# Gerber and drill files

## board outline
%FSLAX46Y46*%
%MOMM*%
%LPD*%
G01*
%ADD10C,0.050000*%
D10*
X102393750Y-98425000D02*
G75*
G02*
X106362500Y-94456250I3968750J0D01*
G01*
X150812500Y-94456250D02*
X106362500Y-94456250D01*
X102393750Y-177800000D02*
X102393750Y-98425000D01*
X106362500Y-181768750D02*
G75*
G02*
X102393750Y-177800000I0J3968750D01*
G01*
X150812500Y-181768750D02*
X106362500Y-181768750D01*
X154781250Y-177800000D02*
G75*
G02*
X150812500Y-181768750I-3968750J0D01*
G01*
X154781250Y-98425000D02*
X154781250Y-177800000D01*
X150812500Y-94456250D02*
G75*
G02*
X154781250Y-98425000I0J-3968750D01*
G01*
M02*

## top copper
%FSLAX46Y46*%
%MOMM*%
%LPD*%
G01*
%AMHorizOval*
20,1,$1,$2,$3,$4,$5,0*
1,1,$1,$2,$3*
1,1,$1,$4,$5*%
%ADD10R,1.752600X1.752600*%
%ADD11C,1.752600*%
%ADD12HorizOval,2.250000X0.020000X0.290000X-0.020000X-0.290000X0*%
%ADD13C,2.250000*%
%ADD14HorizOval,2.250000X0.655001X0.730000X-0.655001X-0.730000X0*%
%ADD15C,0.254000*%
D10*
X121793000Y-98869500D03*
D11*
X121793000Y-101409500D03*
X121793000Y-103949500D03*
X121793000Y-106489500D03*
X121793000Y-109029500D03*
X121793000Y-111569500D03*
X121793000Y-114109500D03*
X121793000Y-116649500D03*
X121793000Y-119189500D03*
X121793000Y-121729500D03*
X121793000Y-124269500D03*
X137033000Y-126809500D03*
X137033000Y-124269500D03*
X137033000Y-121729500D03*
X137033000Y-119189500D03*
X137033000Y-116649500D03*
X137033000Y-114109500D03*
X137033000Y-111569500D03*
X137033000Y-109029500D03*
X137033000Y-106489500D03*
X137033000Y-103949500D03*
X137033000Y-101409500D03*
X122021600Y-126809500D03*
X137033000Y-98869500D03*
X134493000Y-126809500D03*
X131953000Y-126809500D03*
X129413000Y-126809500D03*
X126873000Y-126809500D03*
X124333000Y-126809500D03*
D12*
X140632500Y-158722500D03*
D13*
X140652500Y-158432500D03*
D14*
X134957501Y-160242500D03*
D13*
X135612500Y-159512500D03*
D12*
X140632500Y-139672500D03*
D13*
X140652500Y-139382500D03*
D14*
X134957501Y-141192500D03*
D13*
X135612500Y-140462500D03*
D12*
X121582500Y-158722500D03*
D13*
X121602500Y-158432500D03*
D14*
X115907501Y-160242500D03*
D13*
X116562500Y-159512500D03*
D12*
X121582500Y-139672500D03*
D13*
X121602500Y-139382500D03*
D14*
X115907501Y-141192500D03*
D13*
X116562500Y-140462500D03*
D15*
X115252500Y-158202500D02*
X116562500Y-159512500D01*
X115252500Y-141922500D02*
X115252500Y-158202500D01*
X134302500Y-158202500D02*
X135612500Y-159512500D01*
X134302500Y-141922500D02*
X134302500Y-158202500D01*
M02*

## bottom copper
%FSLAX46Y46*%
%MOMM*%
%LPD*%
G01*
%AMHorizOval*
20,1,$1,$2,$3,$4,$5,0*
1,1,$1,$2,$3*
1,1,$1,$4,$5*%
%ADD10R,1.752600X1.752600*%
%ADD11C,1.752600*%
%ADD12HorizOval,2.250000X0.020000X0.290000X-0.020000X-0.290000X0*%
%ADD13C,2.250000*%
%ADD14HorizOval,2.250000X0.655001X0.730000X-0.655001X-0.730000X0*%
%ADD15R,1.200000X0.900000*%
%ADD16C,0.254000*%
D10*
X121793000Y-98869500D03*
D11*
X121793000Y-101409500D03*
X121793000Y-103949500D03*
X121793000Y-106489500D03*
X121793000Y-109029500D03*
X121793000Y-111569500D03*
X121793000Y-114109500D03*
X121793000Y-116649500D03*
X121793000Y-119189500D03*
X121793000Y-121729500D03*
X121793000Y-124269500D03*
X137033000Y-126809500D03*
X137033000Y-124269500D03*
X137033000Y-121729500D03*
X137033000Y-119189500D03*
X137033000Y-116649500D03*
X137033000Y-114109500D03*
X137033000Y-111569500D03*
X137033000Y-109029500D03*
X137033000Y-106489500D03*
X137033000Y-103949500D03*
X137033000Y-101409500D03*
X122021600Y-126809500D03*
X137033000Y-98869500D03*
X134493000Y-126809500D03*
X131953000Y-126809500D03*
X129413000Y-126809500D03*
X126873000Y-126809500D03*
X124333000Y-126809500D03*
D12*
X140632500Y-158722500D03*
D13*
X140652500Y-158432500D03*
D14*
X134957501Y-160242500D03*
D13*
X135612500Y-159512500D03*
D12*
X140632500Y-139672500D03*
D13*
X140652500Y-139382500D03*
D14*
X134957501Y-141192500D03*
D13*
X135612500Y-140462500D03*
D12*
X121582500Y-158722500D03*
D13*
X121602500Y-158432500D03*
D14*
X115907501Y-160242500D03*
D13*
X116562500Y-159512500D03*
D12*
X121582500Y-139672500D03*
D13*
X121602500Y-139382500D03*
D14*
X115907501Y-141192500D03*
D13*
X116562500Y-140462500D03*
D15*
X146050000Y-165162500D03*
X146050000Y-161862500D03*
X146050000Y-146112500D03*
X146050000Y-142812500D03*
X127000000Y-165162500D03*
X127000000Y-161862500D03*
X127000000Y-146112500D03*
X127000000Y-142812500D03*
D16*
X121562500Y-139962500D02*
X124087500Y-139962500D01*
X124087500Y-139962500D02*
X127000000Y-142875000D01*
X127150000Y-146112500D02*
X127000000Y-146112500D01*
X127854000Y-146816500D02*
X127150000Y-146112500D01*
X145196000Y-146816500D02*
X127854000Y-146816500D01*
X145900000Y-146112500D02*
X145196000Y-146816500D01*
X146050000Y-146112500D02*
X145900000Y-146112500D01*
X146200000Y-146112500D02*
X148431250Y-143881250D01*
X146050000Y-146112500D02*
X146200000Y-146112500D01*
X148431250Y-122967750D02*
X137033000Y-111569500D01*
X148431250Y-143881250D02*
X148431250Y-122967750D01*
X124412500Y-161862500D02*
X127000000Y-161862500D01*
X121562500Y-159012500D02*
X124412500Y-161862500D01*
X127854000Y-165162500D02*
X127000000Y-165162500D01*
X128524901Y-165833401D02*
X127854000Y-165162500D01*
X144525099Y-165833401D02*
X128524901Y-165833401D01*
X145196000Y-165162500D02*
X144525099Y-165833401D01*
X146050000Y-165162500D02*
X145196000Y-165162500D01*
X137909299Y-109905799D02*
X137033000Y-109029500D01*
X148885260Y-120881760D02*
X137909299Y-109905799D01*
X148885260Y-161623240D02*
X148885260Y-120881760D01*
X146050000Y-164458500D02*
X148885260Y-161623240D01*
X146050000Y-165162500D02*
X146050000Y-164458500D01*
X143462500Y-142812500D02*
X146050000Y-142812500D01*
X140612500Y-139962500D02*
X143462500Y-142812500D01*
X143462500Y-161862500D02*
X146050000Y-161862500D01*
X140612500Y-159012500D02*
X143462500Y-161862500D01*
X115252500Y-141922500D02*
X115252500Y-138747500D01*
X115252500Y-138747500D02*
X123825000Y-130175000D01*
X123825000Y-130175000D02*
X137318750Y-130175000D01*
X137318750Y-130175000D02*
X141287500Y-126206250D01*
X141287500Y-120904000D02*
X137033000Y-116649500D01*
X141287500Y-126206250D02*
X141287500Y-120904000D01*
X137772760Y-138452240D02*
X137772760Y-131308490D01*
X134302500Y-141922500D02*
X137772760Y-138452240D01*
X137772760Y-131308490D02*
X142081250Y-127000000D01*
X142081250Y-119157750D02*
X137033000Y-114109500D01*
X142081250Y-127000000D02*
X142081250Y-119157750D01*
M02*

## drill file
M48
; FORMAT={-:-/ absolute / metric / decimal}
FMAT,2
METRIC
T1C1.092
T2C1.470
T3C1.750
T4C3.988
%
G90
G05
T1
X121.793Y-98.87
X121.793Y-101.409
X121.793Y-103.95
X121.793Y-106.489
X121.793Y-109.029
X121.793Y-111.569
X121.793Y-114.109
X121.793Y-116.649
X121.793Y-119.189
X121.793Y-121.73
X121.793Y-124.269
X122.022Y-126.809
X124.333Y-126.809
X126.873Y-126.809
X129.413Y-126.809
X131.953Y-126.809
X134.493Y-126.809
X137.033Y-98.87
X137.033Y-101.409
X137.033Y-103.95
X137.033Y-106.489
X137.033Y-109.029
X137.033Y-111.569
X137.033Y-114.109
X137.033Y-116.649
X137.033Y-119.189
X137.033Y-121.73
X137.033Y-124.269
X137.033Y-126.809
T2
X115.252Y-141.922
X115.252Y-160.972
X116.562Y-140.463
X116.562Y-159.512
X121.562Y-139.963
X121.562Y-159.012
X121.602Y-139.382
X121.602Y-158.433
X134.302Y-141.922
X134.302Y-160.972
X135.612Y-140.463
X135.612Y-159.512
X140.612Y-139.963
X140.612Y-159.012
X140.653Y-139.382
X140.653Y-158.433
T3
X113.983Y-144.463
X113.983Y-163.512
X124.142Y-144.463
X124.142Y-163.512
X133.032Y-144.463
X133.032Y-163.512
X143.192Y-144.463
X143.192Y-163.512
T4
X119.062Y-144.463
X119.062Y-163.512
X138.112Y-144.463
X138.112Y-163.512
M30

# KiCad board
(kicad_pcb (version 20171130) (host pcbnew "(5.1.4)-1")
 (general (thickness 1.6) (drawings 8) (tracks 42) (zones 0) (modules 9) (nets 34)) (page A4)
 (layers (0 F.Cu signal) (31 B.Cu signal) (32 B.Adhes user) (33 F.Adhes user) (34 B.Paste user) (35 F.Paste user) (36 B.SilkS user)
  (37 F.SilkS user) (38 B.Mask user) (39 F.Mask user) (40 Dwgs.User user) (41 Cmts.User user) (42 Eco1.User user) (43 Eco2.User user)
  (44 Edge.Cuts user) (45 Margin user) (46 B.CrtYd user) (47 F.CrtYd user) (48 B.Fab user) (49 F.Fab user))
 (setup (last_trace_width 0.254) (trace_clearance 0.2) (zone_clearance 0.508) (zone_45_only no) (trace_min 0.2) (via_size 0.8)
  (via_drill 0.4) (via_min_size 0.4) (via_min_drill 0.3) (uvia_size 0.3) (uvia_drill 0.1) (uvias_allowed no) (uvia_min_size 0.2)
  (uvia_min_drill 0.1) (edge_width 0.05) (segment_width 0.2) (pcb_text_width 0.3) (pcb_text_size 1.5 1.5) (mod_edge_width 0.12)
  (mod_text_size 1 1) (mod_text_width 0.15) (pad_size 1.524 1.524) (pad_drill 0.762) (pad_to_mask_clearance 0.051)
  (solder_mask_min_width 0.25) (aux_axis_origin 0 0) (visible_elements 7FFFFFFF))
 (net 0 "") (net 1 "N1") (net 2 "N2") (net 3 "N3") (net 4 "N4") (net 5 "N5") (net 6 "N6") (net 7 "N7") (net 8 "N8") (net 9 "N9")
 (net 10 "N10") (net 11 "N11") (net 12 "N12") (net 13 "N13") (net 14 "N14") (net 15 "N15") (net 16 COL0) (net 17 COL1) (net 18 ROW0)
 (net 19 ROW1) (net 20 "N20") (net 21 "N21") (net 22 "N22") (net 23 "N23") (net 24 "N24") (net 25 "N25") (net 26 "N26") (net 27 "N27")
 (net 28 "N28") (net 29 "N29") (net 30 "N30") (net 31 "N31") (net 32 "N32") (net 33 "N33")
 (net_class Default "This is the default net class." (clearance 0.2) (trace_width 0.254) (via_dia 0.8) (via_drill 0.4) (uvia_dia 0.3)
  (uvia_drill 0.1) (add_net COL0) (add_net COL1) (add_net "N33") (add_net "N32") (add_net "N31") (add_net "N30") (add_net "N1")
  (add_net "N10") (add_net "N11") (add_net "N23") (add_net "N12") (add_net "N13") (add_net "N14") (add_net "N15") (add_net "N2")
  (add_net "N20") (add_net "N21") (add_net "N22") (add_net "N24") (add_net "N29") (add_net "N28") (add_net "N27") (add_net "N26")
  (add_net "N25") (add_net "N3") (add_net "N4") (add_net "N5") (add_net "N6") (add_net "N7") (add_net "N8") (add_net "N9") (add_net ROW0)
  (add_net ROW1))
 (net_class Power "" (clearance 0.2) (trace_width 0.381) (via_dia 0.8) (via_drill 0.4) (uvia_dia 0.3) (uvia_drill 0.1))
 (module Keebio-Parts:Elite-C (layer F.Cu) (at 129.413 112.8395 270)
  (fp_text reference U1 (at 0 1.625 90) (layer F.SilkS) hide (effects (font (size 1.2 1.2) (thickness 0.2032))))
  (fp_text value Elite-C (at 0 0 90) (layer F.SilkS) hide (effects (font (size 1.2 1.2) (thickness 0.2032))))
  (pad 1 thru_hole rect (at -13.97 7.62 270) (size 1.7526 1.7526) (drill 1.0922) (layers *.Cu *.SilkS *.Mask) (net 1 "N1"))
  (pad 2 thru_hole circle (at -11.43 7.62 270) (size 1.7526 1.7526) (drill 1.0922) (layers *.Cu *.SilkS *.Mask) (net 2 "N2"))
  (pad 3 thru_hole circle (at -8.89 7.62 270) (size 1.7526 1.7526) (drill 1.0922) (layers *.Cu *.SilkS *.Mask) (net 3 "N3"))
  (pad 4 thru_hole circle (at -6.35 7.62 270) (size 1.7526 1.7526) (drill 1.0922) (layers *.Cu *.SilkS *.Mask) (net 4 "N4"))
  (pad 5 thru_hole circle (at -3.81 7.62 270) (size 1.7526 1.7526) (drill 1.0922) (layers *.Cu *.SilkS *.Mask) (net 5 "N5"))
  (pad 6 thru_hole circle (at -1.27 7.62 270) (size 1.7526 1.7526) (drill 1.0922) (layers *.Cu *.SilkS *.Mask) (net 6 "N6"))
  (pad 7 thru_hole circle (at 1.27 7.62 270) (size 1.7526 1.7526) (drill 1.0922) (layers *.Cu *.SilkS *.Mask) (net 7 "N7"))
  (pad 8 thru_hole circle (at 3.81 7.62 270) (size 1.7526 1.7526) (drill 1.0922) (layers *.Cu *.SilkS *.Mask) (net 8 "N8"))
  (pad 9 thru_hole circle (at 6.35 7.62 270) (size 1.7526 1.7526) (drill 1.0922) (layers *.Cu *.SilkS *.Mask) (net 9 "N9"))
  (pad 10 thru_hole circle (at 8.89 7.62 270) (size 1.7526 1.7526) (drill 1.0922) (layers *.Cu *.SilkS *.Mask) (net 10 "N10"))
  (pad 11 thru_hole circle (at 11.43 7.62 270) (size 1.7526 1.7526) (drill 1.0922) (layers *.Cu *.SilkS *.Mask) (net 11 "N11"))
  (pad 13 thru_hole circle (at 13.97 -7.62 270) (size 1.7526 1.7526) (drill 1.0922) (layers *.Cu *.SilkS *.Mask) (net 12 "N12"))
  (pad 14 thru_hole circle (at 11.43 -7.62 270) (size 1.7526 1.7526) (drill 1.0922) (layers *.Cu *.SilkS *.Mask) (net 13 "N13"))
  (pad 15 thru_hole circle (at 8.89 -7.62 270) (size 1.7526 1.7526) (drill 1.0922) (layers *.Cu *.SilkS *.Mask) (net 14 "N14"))
  (pad 16 thru_hole circle (at 6.35 -7.62 270) (size 1.7526 1.7526) (drill 1.0922) (layers *.Cu *.SilkS *.Mask) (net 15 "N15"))
  (pad 17 thru_hole circle (at 3.81 -7.62 270) (size 1.7526 1.7526) (drill 1.0922) (layers *.Cu *.SilkS *.Mask) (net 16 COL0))
  (pad 18 thru_hole circle (at 1.27 -7.62 270) (size 1.7526 1.7526) (drill 1.0922) (layers *.Cu *.SilkS *.Mask) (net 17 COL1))
  (pad 19 thru_hole circle (at -1.27 -7.62 270) (size 1.7526 1.7526) (drill 1.0922) (layers *.Cu *.SilkS *.Mask) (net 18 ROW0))
  (pad 20 thru_hole circle (at -3.81 -7.62 270) (size 1.7526 1.7526) (drill 1.0922) (layers *.Cu *.SilkS *.Mask) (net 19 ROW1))
  (pad 21 thru_hole circle (at -6.35 -7.62 270) (size 1.7526 1.7526) (drill 1.0922) (layers *.Cu *.SilkS *.Mask) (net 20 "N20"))
  (pad 22 thru_hole circle (at -8.89 -7.62 270) (size 1.7526 1.7526) (drill 1.0922) (layers *.Cu *.SilkS *.Mask) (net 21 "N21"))
  (pad 23 thru_hole circle (at -11.43 -7.62 270) (size 1.7526 1.7526) (drill 1.0922) (layers *.Cu *.SilkS *.Mask) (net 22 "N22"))
  (pad 12 thru_hole circle (at 13.97 7.3914 270) (size 1.7526 1.7526) (drill 1.0922) (layers *.Cu *.SilkS *.Mask) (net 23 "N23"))
  (pad 24 thru_hole circle (at -13.97 -7.62 270) (size 1.7526 1.7526) (drill 1.0922) (layers *.Cu *.SilkS *.Mask) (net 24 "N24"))
  (pad 29 thru_hole circle (at 13.97 -5.08 270) (size 1.7526 1.7526) (drill 1.0922) (layers *.Cu *.SilkS *.Mask) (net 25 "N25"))
  (pad 28 thru_hole circle (at 13.97 -2.54 270) (size 1.7526 1.7526) (drill 1.0922) (layers *.Cu *.SilkS *.Mask) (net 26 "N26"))
  (pad 27 thru_hole circle (at 13.97 0 270) (size 1.7526 1.7526) (drill 1.0922) (layers *.Cu *.SilkS *.Mask) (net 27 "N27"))
  (pad 26 thru_hole circle (at 13.97 2.54 270) (size 1.7526 1.7526) (drill 1.0922) (layers *.Cu *.SilkS *.Mask) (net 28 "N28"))
  (pad 25 thru_hole circle (at 13.97 5.08 270) (size 1.7526 1.7526) (drill 1.0922) (layers *.Cu *.SilkS *.Mask) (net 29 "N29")))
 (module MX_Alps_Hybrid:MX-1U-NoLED (layer F.Cu) (at 138.1125 163.5125)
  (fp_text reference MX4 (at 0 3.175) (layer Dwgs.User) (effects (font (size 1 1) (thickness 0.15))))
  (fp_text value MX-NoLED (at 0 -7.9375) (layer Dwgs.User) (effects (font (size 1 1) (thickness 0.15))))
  (pad 2 thru_hole oval (at 2.5 -4.5 86.0548) (size 2.831378 2.25) (drill 1.47 (offset 0.290689 0)) (layers *.Cu B.Mask) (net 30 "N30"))
  (pad 2 thru_hole circle (at 2.54 -5.08) (size 2.25 2.25) (drill 1.47) (layers *.Cu B.Mask) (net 30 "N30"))
  (pad 1 thru_hole oval (at -3.81 -2.54 48.0996) (size 4.211556 2.25) (drill 1.47 (offset 0.980778 0)) (layers *.Cu B.Mask) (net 17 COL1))
  (pad "" np_thru_hole circle (at 0 0) (size 3.9878 3.9878) (drill 3.9878) (layers *.Cu *.Mask))
  (pad 1 thru_hole circle (at -2.5 -4) (size 2.25 2.25) (drill 1.47) (layers *.Cu B.Mask) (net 17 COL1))
  (pad "" np_thru_hole circle (at -5.08 0 48.0996) (size 1.75 1.75) (drill 1.75) (layers *.Cu *.Mask))
  (pad "" np_thru_hole circle (at 5.08 0 48.0996) (size 1.75 1.75) (drill 1.75) (layers *.Cu *.Mask)))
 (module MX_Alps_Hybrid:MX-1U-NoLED (layer F.Cu) (at 138.1125 144.4625)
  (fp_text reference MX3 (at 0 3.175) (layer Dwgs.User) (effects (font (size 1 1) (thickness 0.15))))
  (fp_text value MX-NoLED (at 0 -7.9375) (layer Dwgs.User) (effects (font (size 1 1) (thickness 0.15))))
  (pad 2 thru_hole oval (at 2.5 -4.5 86.0548) (size 2.831378 2.25) (drill 1.47 (offset 0.290689 0)) (layers *.Cu B.Mask) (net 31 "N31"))
  (pad 2 thru_hole circle (at 2.54 -5.08) (size 2.25 2.25) (drill 1.47) (layers *.Cu B.Mask) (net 31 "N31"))
  (pad 1 thru_hole oval (at -3.81 -2.54 48.0996) (size 4.211556 2.25) (drill 1.47 (offset 0.980778 0)) (layers *.Cu B.Mask) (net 17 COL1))
  (pad "" np_thru_hole circle (at 0 0) (size 3.9878 3.9878) (drill 3.9878) (layers *.Cu *.Mask))
  (pad 1 thru_hole circle (at -2.5 -4) (size 2.25 2.25) (drill 1.47) (layers *.Cu B.Mask) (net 17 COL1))
  (pad "" np_thru_hole circle (at -5.08 0 48.0996) (size 1.75 1.75) (drill 1.75) (layers *.Cu *.Mask))
  (pad "" np_thru_hole circle (at 5.08 0 48.0996) (size 1.75 1.75) (drill 1.75) (layers *.Cu *.Mask)))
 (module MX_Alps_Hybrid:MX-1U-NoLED (layer F.Cu) (at 119.0625 163.5125)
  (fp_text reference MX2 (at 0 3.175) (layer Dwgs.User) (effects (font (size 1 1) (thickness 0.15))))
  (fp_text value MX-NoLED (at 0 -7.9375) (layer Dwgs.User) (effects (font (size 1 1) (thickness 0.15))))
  (pad 2 thru_hole oval (at 2.5 -4.5 86.0548) (size 2.831378 2.25) (drill 1.47 (offset 0.290689 0)) (layers *.Cu B.Mask) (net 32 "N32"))
  (pad 2 thru_hole circle (at 2.54 -5.08) (size 2.25 2.25) (drill 1.47) (layers *.Cu B.Mask) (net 32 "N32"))
  (pad 1 thru_hole oval (at -3.81 -2.54 48.0996) (size 4.211556 2.25) (drill 1.47 (offset 0.980778 0)) (layers *.Cu B.Mask) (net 16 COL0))
  (pad "" np_thru_hole circle (at 0 0) (size 3.9878 3.9878) (drill 3.9878) (layers *.Cu *.Mask))
  (pad 1 thru_hole circle (at -2.5 -4) (size 2.25 2.25) (drill 1.47) (layers *.Cu B.Mask) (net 16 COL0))
  (pad "" np_thru_hole circle (at -5.08 0 48.0996) (size 1.75 1.75) (drill 1.75) (layers *.Cu *.Mask))
  (pad "" np_thru_hole circle (at 5.08 0 48.0996) (size 1.75 1.75) (drill 1.75) (layers *.Cu *.Mask)))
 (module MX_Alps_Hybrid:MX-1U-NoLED (layer F.Cu) (at 119.0625 144.4625)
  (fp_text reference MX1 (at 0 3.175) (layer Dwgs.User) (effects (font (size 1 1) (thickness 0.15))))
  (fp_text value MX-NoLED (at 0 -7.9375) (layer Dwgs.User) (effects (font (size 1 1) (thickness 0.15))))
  (pad 2 thru_hole oval (at 2.5 -4.5 86.0548) (size 2.831378 2.25) (drill 1.47 (offset 0.290689 0)) (layers *.Cu B.Mask) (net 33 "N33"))
  (pad 2 thru_hole circle (at 2.54 -5.08) (size 2.25 2.25) (drill 1.47) (layers *.Cu B.Mask) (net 33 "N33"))
  (pad 1 thru_hole oval (at -3.81 -2.54 48.0996) (size 4.211556 2.25) (drill 1.47 (offset 0.980778 0)) (layers *.Cu B.Mask) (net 16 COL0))
  (pad "" np_thru_hole circle (at 0 0) (size 3.9878 3.9878) (drill 3.9878) (layers *.Cu *.Mask))
  (pad 1 thru_hole circle (at -2.5 -4) (size 2.25 2.25) (drill 1.47) (layers *.Cu B.Mask) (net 16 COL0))
  (pad "" np_thru_hole circle (at -5.08 0 48.0996) (size 1.75 1.75) (drill 1.75) (layers *.Cu *.Mask))
  (pad "" np_thru_hole circle (at 5.08 0 48.0996) (size 1.75 1.75) (drill 1.75) (layers *.Cu *.Mask)))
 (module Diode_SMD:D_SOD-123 (layer B.Cu) (at 146.05 163.5125 90)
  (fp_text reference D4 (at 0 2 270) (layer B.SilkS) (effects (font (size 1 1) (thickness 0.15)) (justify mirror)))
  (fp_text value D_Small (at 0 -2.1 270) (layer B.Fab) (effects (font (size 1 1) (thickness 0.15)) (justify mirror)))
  (pad 1 smd rect (at -1.65 0 90) (size 0.9 1.2) (layers B.Cu B.Paste B.Mask) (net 19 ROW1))
  (pad 2 smd rect (at 1.65 0 90) (size 0.9 1.2) (layers B.Cu B.Paste B.Mask) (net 30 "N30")))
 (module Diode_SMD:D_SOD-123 (layer B.Cu) (at 146.05 144.4625 90)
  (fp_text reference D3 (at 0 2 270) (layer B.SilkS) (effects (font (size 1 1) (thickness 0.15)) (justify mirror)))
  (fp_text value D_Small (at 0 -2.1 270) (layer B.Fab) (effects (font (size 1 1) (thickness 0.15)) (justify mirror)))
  (pad 1 smd rect (at -1.65 0 90) (size 0.9 1.2) (layers B.Cu B.Paste B.Mask) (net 18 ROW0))
  (pad 2 smd rect (at 1.65 0 90) (size 0.9 1.2) (layers B.Cu B.Paste B.Mask) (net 31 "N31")))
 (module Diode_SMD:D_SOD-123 (layer B.Cu) (at 127 163.5125 90)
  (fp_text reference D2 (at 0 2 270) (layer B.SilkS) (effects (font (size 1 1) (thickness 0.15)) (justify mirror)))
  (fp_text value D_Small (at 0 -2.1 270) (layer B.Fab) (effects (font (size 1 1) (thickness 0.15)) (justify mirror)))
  (pad 1 smd rect (at -1.65 0 90) (size 0.9 1.2) (layers B.Cu B.Paste B.Mask) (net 19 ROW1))
  (pad 2 smd rect (at 1.65 0 90) (size 0.9 1.2) (layers B.Cu B.Paste B.Mask) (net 32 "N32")))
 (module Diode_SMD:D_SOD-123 (layer B.Cu) (at 127 144.4625 90)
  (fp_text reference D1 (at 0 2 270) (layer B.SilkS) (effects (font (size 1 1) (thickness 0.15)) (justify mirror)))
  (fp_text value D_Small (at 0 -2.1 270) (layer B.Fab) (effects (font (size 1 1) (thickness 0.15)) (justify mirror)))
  (pad 1 smd rect (at -1.65 0 90) (size 0.9 1.2) (layers B.Cu B.Paste B.Mask) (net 18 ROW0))
  (pad 2 smd rect (at 1.65 0 90) (size 0.9 1.2) (layers B.Cu B.Paste B.Mask) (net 33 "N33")))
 (gr_arc (start 106.3625 98.425) (end 106.3625 94.45625) (angle -90) (layer Edge.Cuts) (width 0.05))
 (gr_line (start 150.8125 94.45625) (end 106.3625 94.45625) (layer Edge.Cuts) (width 0.05))
 (gr_line (start 102.39375 177.8) (end 102.39375 98.425) (layer Edge.Cuts) (width 0.05))
 (gr_arc (start 106.3625 177.8) (end 102.39375 177.8) (angle -90) (layer Edge.Cuts) (width 0.05))
 (gr_line (start 150.8125 181.76875) (end 106.3625 181.76875) (layer Edge.Cuts) (width 0.05))
 (gr_arc (start 150.8125 177.8) (end 150.8125 181.76875) (angle -90) (layer Edge.Cuts) (width 0.05))
 (gr_line (start 154.78125 98.425) (end 154.78125 177.8) (layer Edge.Cuts) (width 0.05))
 (gr_arc (start 150.8125 98.425) (end 154.78125 98.425) (angle -90) (layer Edge.Cuts) (width 0.05))
 (segment (start 121.5625 139.9625) (end 124.0875 139.9625) (width 0.254) (layer B.Cu) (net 33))
 (segment (start 124.0875 139.9625) (end 127 142.875) (width 0.254) (layer B.Cu) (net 33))
 (segment (start 127.15 146.1125) (end 127 146.1125) (width 0.254) (layer B.Cu) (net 18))
 (segment (start 127.854 146.8165) (end 127.15 146.1125) (width 0.254) (layer B.Cu) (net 18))
 (segment (start 145.196 146.8165) (end 127.854 146.8165) (width 0.254) (layer B.Cu) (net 18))
 (segment (start 145.9 146.1125) (end 145.196 146.8165) (width 0.254) (layer B.Cu) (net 18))
 (segment (start 146.05 146.1125) (end 145.9 146.1125) (width 0.254) (layer B.Cu) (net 18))
 (segment (start 146.2 146.1125) (end 148.43125 143.88125) (width 0.254) (layer B.Cu) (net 18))
 (segment (start 146.05 146.1125) (end 146.2 146.1125) (width 0.254) (layer B.Cu) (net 18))
 (segment (start 148.43125 122.96775) (end 137.033 111.5695) (width 0.254) (layer B.Cu) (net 18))
 (segment (start 148.43125 143.88125) (end 148.43125 122.96775) (width 0.254) (layer B.Cu) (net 18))
 (segment (start 124.4125 161.8625) (end 127 161.8625) (width 0.254) (layer B.Cu) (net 32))
 (segment (start 121.5625 159.0125) (end 124.4125 161.8625) (width 0.254) (layer B.Cu) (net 32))
 (segment (start 127.854 165.1625) (end 127 165.1625) (width 0.254) (layer B.Cu) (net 19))
 (segment (start 128.524901 165.833401) (end 127.854 165.1625) (width 0.254) (layer B.Cu) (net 19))
 (segment (start 144.525099 165.833401) (end 128.524901 165.833401) (width 0.254) (layer B.Cu) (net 19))
 (segment (start 145.196 165.1625) (end 144.525099 165.833401) (width 0.254) (layer B.Cu) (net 19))
 (segment (start 146.05 165.1625) (end 145.196 165.1625) (width 0.254) (layer B.Cu) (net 19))
 (segment (start 137.909299 109.905799) (end 137.033 109.0295) (width 0.254) (layer B.Cu) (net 19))
 (segment (start 148.88526 120.88176) (end 137.909299 109.905799) (width 0.254) (layer B.Cu) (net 19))
 (segment (start 148.88526 161.62324) (end 148.88526 120.88176) (width 0.254) (layer B.Cu) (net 19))
 (segment (start 146.05 164.4585) (end 148.88526 161.62324) (width 0.254) (layer B.Cu) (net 19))
 (segment (start 146.05 165.1625) (end 146.05 164.4585) (width 0.254) (layer B.Cu) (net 19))
 (segment (start 143.4625 142.8125) (end 146.05 142.8125) (width 0.254) (layer B.Cu) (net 31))
 (segment (start 140.6125 139.9625) (end 143.4625 142.8125) (width 0.254) (layer B.Cu) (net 31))
 (segment (start 143.4625 161.8625) (end 146.05 161.8625) (width 0.254) (layer B.Cu) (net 30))
 (segment (start 140.6125 159.0125) (end 143.4625 161.8625) (width 0.254) (layer B.Cu) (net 30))
 (segment (start 115.2525 158.2025) (end 116.5625 159.5125) (width 0.254) (layer F.Cu) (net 16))
 (segment (start 115.2525 141.9225) (end 115.2525 158.2025) (width 0.254) (layer F.Cu) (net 16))
 (segment (start 115.2525 141.9225) (end 115.2525 138.7475) (width 0.254) (layer B.Cu) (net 16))
 (segment (start 115.2525 138.7475) (end 123.825 130.175) (width 0.254) (layer B.Cu) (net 16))
 (segment (start 123.825 130.175) (end 137.31875 130.175) (width 0.254) (layer B.Cu) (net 16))
 (segment (start 137.31875 130.175) (end 141.2875 126.20625) (width 0.254) (layer B.Cu) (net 16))
 (segment (start 141.2875 120.904) (end 137.033 116.6495) (width 0.254) (layer B.Cu) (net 16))
 (segment (start 141.2875 126.20625) (end 141.2875 120.904) (width 0.254) (layer B.Cu) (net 16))
 (segment (start 134.3025 158.2025) (end 135.6125 159.5125) (width 0.254) (layer F.Cu) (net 17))
 (segment (start 134.3025 141.9225) (end 134.3025 158.2025) (width 0.254) (layer F.Cu) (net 17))
 (segment (start 137.77276 138.45224) (end 137.77276 131.30849) (width 0.254) (layer B.Cu) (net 17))
 (segment (start 134.3025 141.9225) (end 137.77276 138.45224) (width 0.254) (layer B.Cu) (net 17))
 (segment (start 137.77276 131.30849) (end 142.08125 127) (width 0.254) (layer B.Cu) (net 17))
 (segment (start 142.08125 119.15775) (end 137.033 114.1095) (width 0.254) (layer B.Cu) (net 17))
 (segment (start 142.08125 127) (end 142.08125 119.15775) (width 0.254) (layer B.Cu) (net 17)))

